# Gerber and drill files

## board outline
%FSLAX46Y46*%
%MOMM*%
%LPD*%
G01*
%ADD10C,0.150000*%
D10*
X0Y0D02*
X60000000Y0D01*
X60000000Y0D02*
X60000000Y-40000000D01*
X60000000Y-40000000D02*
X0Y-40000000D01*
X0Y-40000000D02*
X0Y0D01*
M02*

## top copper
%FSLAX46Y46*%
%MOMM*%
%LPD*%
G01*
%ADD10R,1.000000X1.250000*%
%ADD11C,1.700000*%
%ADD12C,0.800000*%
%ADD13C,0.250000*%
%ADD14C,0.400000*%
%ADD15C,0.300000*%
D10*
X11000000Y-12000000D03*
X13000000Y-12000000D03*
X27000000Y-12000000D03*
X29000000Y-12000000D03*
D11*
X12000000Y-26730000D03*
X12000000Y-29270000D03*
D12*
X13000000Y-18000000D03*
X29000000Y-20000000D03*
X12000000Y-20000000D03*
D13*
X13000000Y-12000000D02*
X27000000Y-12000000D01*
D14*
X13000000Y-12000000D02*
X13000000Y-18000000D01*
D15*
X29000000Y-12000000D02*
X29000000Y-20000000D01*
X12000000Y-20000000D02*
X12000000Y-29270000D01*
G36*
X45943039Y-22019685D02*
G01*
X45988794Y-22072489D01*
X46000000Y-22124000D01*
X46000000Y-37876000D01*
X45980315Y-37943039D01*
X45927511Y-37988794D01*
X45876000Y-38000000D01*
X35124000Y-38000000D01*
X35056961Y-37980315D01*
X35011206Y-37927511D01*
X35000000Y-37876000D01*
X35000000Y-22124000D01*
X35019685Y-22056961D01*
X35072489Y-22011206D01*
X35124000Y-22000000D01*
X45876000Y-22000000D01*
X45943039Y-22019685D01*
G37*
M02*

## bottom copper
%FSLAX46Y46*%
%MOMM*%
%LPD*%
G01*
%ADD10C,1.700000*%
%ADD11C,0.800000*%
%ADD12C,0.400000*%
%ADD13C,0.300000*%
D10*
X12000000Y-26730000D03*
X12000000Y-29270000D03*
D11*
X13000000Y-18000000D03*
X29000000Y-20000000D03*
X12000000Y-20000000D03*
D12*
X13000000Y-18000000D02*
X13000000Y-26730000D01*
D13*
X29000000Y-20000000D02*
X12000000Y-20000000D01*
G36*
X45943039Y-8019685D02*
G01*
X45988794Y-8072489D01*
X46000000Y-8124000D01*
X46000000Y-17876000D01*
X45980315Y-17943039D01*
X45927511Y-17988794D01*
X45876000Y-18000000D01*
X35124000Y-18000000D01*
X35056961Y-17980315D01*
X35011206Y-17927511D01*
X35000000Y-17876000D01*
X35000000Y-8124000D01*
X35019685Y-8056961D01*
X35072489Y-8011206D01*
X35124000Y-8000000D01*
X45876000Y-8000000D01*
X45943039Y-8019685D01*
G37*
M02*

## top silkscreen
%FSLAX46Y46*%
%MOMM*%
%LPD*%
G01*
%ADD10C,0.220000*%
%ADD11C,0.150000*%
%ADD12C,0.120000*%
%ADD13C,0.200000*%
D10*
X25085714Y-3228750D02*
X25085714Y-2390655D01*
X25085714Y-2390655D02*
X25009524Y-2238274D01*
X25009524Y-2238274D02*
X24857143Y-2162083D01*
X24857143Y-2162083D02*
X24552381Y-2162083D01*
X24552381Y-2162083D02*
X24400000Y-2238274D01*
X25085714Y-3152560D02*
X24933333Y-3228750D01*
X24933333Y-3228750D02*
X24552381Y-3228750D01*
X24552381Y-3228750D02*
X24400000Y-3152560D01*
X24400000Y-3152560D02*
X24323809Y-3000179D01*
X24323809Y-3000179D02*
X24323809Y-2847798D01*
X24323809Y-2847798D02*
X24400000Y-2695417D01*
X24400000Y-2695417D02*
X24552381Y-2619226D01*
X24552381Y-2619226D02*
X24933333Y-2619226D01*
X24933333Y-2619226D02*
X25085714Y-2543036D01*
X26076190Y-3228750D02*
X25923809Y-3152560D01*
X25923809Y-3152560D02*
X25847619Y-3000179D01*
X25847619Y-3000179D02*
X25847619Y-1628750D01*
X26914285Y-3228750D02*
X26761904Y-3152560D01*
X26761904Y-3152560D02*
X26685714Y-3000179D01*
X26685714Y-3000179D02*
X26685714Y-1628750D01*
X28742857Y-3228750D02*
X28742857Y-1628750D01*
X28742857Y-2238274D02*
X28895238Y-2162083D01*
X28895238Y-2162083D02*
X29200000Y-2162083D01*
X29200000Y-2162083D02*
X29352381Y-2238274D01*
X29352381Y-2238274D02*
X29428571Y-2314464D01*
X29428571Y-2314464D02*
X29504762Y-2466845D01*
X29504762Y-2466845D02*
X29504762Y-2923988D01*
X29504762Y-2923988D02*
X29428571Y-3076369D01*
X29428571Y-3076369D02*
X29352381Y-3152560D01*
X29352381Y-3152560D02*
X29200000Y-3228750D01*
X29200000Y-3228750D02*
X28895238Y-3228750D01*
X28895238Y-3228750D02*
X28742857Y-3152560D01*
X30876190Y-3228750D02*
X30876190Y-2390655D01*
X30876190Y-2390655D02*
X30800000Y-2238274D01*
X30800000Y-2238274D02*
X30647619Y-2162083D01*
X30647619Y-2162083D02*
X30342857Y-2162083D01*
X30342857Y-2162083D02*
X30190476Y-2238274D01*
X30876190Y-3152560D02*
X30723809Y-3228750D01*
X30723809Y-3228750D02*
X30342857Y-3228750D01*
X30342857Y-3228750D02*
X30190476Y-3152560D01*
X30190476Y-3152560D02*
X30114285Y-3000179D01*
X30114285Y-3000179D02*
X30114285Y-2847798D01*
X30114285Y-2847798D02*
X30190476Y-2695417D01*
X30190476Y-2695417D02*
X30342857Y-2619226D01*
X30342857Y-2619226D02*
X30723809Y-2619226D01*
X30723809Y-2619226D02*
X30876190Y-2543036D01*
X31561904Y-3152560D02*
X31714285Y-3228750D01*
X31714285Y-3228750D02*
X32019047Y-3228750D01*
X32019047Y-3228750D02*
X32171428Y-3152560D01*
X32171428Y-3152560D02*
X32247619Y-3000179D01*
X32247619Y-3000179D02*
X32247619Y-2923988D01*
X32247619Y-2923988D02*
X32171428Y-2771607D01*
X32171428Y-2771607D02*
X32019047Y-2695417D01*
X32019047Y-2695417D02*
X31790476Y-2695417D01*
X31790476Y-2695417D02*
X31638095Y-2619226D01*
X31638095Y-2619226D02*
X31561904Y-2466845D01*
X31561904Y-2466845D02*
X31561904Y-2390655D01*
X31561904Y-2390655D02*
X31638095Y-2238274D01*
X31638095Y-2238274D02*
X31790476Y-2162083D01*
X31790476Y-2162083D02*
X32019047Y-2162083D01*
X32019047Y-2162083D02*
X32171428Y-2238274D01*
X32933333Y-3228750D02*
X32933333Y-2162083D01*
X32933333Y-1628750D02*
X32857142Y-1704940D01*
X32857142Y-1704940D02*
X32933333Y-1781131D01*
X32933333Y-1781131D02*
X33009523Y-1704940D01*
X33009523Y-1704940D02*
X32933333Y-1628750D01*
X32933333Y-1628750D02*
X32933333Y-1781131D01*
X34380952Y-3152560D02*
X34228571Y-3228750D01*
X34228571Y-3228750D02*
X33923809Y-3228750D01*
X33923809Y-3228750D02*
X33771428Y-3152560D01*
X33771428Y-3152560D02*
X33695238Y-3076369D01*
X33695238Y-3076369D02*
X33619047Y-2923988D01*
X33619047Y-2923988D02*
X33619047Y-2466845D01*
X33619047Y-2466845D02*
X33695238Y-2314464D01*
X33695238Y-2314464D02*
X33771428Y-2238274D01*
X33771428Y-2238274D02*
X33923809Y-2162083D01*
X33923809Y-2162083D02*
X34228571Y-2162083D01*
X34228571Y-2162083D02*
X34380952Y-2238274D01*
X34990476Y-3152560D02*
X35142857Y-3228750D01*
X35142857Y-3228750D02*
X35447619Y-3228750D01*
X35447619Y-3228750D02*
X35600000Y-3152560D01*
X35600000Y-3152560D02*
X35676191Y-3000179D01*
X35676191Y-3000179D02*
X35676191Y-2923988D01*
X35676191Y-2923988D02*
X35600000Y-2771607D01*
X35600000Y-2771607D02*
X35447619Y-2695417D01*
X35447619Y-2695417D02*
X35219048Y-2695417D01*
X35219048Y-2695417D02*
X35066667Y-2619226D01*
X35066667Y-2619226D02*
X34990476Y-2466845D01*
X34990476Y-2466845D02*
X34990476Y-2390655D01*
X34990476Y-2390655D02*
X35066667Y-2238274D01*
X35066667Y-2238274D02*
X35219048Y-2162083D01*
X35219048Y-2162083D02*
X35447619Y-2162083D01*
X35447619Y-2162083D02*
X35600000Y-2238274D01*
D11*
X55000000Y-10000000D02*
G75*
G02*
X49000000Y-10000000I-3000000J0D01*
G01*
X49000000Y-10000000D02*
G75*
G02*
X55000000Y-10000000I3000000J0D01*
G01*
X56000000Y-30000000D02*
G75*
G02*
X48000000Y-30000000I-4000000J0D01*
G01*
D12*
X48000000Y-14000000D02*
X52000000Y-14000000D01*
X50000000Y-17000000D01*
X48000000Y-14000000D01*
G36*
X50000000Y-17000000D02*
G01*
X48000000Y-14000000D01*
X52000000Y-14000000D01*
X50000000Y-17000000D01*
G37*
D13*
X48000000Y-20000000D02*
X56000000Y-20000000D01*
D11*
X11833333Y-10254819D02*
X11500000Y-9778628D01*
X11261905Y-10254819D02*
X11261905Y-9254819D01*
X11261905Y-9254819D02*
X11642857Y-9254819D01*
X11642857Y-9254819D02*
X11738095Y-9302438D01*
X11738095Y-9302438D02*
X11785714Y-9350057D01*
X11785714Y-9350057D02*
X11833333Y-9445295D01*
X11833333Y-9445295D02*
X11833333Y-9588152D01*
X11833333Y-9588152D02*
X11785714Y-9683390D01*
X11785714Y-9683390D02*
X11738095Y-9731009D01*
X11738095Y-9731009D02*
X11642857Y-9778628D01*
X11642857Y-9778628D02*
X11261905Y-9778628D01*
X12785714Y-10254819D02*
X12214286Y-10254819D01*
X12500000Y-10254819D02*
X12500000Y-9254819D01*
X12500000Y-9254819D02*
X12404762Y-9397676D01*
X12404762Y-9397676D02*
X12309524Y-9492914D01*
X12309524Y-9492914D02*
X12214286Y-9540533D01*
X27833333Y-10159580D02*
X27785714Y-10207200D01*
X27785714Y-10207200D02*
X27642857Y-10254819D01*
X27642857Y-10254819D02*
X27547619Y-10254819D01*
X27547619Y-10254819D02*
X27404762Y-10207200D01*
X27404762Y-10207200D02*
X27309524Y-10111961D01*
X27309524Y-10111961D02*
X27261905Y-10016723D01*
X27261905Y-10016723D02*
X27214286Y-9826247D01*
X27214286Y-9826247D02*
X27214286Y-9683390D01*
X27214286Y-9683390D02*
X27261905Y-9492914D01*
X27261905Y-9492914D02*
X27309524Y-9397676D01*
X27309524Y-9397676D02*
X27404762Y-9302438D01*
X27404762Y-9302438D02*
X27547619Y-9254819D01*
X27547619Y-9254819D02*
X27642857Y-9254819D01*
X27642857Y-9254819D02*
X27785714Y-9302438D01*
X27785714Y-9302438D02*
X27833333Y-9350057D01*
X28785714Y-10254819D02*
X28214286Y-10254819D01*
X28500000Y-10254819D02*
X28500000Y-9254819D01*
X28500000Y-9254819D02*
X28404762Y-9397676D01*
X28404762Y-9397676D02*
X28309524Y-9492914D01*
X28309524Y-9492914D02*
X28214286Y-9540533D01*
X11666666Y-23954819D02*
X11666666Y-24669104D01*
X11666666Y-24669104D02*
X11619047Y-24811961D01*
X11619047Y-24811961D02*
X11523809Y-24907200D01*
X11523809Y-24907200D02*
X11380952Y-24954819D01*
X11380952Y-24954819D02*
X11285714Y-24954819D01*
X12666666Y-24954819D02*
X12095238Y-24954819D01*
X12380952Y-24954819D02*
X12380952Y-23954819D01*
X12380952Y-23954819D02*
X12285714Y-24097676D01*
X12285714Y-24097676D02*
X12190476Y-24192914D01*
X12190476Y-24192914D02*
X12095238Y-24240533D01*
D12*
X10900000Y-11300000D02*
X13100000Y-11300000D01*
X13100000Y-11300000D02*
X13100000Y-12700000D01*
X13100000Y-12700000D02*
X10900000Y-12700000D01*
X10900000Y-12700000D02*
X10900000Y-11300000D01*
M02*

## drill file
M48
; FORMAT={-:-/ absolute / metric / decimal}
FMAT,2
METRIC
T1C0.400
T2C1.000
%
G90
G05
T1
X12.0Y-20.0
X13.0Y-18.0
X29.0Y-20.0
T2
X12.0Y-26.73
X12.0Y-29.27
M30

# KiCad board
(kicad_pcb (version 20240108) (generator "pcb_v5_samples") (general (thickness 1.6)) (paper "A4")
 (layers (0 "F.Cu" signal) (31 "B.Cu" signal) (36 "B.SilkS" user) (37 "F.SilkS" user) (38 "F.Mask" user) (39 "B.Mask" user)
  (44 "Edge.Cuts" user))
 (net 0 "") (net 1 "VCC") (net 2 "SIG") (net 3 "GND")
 (gr_line (start 0 0) (end 60 0) (stroke (width 0.15) (type solid)) (layer "Edge.Cuts"))
 (gr_line (start 60 0) (end 60 40) (stroke (width 0.15) (type solid)) (layer "Edge.Cuts"))
 (gr_line (start 60 40) (end 0 40) (stroke (width 0.15) (type solid)) (layer "Edge.Cuts"))
 (gr_line (start 0 40) (end 0 0) (stroke (width 0.15) (type solid)) (layer "Edge.Cuts"))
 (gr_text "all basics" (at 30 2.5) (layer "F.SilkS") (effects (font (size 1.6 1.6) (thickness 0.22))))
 (gr_circle (center 52 10) (end 55 10) (stroke (width 0.15) (type solid)) (fill no) (layer "F.SilkS"))
 (gr_arc (start 48 30) (mid 52 34) (end 56 30) (stroke (width 0.15) (type solid)) (layer "F.SilkS"))
 (gr_poly (pts (xy 48 14) (xy 52 14) (xy 50 17)) (stroke (width 0.12) (type solid)) (fill yes) (layer "F.SilkS"))
 (gr_line (start 48 20) (end 56 20) (stroke (width 0.2) (type solid)) (layer "F.SilkS"))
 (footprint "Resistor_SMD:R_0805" (layer "F.Cu") (at 12 12)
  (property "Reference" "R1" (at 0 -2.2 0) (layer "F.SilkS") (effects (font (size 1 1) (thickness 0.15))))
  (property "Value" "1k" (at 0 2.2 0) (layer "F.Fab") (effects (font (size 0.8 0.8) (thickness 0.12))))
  (fp_line (start -1.1 -0.7) (end 1.1 -0.7) (stroke (width 0.12) (type solid)) (layer "F.SilkS"))
  (fp_line (start 1.1 -0.7) (end 1.1 0.7) (stroke (width 0.12) (type solid)) (layer "F.SilkS"))
  (fp_line (start 1.1 0.7) (end -1.1 0.7) (stroke (width 0.12) (type solid)) (layer "F.SilkS"))
  (fp_line (start -1.1 0.7) (end -1.1 -0.7) (stroke (width 0.12) (type solid)) (layer "F.SilkS"))
  (pad "1" smd rect (at -1.0 0) (size 1.0 1.25) (layers "F.Cu" "F.Paste" "F.Mask") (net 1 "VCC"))
  (pad "2" smd rect (at 1.0 0) (size 1.0 1.25) (layers "F.Cu" "F.Paste" "F.Mask") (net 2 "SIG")))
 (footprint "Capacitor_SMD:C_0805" (layer "F.Cu") (at 28 12)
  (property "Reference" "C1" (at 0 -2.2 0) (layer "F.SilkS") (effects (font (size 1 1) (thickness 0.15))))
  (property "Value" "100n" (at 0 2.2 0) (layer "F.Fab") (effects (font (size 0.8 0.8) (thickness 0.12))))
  (pad "1" smd rect (at -1.0 0) (size 1.0 1.25) (layers "F.Cu" "F.Paste" "F.Mask") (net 2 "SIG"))
  (pad "2" smd rect (at 1.0 0) (size 1.0 1.25) (layers "F.Cu" "F.Paste" "F.Mask") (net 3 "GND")))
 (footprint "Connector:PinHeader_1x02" (layer "F.Cu") (at 12 28)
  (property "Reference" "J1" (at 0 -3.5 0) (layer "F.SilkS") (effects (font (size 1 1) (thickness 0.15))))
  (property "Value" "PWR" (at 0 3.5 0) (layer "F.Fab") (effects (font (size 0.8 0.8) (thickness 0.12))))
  (pad "1" thru_hole circle (at 0 -1.27) (size 1.7 1.7) (drill 1.0) (layers "*.Cu" "*.Mask") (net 1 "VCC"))
  (pad "2" thru_hole circle (at 0 1.27) (size 1.7 1.7) (drill 1.0) (layers "*.Cu" "*.Mask") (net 3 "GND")))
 (segment (start 13 12) (end 27 12) (width 0.25) (layer "F.Cu") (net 2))
 (segment (start 13 12) (end 13 18) (width 0.4) (layer "F.Cu") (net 1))
 (via (at 13 18) (size 0.8) (drill 0.4) (layers "F.Cu" "B.Cu") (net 1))
 (segment (start 13 18) (end 13 26.73) (width 0.4) (layer "B.Cu") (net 1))
 (segment (start 29 12) (end 29 20) (width 0.3) (layer "F.Cu") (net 3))
 (via (at 29 20) (size 0.8) (drill 0.4) (layers "F.Cu" "B.Cu") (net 3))
 (segment (start 29 20) (end 12 20) (width 0.3) (layer "B.Cu") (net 3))
 (via (at 12 20) (size 0.8) (drill 0.4) (layers "F.Cu" "B.Cu") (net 3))
 (segment (start 12 20) (end 12 29.27) (width 0.3) (layer "F.Cu") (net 3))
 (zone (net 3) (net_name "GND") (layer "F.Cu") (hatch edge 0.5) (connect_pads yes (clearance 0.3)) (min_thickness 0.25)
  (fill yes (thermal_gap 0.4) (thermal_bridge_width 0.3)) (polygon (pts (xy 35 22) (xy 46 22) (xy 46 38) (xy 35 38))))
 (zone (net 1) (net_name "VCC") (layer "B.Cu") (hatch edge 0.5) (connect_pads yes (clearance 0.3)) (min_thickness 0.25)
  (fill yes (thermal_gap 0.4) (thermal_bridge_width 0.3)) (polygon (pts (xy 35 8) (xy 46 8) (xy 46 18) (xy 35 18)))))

